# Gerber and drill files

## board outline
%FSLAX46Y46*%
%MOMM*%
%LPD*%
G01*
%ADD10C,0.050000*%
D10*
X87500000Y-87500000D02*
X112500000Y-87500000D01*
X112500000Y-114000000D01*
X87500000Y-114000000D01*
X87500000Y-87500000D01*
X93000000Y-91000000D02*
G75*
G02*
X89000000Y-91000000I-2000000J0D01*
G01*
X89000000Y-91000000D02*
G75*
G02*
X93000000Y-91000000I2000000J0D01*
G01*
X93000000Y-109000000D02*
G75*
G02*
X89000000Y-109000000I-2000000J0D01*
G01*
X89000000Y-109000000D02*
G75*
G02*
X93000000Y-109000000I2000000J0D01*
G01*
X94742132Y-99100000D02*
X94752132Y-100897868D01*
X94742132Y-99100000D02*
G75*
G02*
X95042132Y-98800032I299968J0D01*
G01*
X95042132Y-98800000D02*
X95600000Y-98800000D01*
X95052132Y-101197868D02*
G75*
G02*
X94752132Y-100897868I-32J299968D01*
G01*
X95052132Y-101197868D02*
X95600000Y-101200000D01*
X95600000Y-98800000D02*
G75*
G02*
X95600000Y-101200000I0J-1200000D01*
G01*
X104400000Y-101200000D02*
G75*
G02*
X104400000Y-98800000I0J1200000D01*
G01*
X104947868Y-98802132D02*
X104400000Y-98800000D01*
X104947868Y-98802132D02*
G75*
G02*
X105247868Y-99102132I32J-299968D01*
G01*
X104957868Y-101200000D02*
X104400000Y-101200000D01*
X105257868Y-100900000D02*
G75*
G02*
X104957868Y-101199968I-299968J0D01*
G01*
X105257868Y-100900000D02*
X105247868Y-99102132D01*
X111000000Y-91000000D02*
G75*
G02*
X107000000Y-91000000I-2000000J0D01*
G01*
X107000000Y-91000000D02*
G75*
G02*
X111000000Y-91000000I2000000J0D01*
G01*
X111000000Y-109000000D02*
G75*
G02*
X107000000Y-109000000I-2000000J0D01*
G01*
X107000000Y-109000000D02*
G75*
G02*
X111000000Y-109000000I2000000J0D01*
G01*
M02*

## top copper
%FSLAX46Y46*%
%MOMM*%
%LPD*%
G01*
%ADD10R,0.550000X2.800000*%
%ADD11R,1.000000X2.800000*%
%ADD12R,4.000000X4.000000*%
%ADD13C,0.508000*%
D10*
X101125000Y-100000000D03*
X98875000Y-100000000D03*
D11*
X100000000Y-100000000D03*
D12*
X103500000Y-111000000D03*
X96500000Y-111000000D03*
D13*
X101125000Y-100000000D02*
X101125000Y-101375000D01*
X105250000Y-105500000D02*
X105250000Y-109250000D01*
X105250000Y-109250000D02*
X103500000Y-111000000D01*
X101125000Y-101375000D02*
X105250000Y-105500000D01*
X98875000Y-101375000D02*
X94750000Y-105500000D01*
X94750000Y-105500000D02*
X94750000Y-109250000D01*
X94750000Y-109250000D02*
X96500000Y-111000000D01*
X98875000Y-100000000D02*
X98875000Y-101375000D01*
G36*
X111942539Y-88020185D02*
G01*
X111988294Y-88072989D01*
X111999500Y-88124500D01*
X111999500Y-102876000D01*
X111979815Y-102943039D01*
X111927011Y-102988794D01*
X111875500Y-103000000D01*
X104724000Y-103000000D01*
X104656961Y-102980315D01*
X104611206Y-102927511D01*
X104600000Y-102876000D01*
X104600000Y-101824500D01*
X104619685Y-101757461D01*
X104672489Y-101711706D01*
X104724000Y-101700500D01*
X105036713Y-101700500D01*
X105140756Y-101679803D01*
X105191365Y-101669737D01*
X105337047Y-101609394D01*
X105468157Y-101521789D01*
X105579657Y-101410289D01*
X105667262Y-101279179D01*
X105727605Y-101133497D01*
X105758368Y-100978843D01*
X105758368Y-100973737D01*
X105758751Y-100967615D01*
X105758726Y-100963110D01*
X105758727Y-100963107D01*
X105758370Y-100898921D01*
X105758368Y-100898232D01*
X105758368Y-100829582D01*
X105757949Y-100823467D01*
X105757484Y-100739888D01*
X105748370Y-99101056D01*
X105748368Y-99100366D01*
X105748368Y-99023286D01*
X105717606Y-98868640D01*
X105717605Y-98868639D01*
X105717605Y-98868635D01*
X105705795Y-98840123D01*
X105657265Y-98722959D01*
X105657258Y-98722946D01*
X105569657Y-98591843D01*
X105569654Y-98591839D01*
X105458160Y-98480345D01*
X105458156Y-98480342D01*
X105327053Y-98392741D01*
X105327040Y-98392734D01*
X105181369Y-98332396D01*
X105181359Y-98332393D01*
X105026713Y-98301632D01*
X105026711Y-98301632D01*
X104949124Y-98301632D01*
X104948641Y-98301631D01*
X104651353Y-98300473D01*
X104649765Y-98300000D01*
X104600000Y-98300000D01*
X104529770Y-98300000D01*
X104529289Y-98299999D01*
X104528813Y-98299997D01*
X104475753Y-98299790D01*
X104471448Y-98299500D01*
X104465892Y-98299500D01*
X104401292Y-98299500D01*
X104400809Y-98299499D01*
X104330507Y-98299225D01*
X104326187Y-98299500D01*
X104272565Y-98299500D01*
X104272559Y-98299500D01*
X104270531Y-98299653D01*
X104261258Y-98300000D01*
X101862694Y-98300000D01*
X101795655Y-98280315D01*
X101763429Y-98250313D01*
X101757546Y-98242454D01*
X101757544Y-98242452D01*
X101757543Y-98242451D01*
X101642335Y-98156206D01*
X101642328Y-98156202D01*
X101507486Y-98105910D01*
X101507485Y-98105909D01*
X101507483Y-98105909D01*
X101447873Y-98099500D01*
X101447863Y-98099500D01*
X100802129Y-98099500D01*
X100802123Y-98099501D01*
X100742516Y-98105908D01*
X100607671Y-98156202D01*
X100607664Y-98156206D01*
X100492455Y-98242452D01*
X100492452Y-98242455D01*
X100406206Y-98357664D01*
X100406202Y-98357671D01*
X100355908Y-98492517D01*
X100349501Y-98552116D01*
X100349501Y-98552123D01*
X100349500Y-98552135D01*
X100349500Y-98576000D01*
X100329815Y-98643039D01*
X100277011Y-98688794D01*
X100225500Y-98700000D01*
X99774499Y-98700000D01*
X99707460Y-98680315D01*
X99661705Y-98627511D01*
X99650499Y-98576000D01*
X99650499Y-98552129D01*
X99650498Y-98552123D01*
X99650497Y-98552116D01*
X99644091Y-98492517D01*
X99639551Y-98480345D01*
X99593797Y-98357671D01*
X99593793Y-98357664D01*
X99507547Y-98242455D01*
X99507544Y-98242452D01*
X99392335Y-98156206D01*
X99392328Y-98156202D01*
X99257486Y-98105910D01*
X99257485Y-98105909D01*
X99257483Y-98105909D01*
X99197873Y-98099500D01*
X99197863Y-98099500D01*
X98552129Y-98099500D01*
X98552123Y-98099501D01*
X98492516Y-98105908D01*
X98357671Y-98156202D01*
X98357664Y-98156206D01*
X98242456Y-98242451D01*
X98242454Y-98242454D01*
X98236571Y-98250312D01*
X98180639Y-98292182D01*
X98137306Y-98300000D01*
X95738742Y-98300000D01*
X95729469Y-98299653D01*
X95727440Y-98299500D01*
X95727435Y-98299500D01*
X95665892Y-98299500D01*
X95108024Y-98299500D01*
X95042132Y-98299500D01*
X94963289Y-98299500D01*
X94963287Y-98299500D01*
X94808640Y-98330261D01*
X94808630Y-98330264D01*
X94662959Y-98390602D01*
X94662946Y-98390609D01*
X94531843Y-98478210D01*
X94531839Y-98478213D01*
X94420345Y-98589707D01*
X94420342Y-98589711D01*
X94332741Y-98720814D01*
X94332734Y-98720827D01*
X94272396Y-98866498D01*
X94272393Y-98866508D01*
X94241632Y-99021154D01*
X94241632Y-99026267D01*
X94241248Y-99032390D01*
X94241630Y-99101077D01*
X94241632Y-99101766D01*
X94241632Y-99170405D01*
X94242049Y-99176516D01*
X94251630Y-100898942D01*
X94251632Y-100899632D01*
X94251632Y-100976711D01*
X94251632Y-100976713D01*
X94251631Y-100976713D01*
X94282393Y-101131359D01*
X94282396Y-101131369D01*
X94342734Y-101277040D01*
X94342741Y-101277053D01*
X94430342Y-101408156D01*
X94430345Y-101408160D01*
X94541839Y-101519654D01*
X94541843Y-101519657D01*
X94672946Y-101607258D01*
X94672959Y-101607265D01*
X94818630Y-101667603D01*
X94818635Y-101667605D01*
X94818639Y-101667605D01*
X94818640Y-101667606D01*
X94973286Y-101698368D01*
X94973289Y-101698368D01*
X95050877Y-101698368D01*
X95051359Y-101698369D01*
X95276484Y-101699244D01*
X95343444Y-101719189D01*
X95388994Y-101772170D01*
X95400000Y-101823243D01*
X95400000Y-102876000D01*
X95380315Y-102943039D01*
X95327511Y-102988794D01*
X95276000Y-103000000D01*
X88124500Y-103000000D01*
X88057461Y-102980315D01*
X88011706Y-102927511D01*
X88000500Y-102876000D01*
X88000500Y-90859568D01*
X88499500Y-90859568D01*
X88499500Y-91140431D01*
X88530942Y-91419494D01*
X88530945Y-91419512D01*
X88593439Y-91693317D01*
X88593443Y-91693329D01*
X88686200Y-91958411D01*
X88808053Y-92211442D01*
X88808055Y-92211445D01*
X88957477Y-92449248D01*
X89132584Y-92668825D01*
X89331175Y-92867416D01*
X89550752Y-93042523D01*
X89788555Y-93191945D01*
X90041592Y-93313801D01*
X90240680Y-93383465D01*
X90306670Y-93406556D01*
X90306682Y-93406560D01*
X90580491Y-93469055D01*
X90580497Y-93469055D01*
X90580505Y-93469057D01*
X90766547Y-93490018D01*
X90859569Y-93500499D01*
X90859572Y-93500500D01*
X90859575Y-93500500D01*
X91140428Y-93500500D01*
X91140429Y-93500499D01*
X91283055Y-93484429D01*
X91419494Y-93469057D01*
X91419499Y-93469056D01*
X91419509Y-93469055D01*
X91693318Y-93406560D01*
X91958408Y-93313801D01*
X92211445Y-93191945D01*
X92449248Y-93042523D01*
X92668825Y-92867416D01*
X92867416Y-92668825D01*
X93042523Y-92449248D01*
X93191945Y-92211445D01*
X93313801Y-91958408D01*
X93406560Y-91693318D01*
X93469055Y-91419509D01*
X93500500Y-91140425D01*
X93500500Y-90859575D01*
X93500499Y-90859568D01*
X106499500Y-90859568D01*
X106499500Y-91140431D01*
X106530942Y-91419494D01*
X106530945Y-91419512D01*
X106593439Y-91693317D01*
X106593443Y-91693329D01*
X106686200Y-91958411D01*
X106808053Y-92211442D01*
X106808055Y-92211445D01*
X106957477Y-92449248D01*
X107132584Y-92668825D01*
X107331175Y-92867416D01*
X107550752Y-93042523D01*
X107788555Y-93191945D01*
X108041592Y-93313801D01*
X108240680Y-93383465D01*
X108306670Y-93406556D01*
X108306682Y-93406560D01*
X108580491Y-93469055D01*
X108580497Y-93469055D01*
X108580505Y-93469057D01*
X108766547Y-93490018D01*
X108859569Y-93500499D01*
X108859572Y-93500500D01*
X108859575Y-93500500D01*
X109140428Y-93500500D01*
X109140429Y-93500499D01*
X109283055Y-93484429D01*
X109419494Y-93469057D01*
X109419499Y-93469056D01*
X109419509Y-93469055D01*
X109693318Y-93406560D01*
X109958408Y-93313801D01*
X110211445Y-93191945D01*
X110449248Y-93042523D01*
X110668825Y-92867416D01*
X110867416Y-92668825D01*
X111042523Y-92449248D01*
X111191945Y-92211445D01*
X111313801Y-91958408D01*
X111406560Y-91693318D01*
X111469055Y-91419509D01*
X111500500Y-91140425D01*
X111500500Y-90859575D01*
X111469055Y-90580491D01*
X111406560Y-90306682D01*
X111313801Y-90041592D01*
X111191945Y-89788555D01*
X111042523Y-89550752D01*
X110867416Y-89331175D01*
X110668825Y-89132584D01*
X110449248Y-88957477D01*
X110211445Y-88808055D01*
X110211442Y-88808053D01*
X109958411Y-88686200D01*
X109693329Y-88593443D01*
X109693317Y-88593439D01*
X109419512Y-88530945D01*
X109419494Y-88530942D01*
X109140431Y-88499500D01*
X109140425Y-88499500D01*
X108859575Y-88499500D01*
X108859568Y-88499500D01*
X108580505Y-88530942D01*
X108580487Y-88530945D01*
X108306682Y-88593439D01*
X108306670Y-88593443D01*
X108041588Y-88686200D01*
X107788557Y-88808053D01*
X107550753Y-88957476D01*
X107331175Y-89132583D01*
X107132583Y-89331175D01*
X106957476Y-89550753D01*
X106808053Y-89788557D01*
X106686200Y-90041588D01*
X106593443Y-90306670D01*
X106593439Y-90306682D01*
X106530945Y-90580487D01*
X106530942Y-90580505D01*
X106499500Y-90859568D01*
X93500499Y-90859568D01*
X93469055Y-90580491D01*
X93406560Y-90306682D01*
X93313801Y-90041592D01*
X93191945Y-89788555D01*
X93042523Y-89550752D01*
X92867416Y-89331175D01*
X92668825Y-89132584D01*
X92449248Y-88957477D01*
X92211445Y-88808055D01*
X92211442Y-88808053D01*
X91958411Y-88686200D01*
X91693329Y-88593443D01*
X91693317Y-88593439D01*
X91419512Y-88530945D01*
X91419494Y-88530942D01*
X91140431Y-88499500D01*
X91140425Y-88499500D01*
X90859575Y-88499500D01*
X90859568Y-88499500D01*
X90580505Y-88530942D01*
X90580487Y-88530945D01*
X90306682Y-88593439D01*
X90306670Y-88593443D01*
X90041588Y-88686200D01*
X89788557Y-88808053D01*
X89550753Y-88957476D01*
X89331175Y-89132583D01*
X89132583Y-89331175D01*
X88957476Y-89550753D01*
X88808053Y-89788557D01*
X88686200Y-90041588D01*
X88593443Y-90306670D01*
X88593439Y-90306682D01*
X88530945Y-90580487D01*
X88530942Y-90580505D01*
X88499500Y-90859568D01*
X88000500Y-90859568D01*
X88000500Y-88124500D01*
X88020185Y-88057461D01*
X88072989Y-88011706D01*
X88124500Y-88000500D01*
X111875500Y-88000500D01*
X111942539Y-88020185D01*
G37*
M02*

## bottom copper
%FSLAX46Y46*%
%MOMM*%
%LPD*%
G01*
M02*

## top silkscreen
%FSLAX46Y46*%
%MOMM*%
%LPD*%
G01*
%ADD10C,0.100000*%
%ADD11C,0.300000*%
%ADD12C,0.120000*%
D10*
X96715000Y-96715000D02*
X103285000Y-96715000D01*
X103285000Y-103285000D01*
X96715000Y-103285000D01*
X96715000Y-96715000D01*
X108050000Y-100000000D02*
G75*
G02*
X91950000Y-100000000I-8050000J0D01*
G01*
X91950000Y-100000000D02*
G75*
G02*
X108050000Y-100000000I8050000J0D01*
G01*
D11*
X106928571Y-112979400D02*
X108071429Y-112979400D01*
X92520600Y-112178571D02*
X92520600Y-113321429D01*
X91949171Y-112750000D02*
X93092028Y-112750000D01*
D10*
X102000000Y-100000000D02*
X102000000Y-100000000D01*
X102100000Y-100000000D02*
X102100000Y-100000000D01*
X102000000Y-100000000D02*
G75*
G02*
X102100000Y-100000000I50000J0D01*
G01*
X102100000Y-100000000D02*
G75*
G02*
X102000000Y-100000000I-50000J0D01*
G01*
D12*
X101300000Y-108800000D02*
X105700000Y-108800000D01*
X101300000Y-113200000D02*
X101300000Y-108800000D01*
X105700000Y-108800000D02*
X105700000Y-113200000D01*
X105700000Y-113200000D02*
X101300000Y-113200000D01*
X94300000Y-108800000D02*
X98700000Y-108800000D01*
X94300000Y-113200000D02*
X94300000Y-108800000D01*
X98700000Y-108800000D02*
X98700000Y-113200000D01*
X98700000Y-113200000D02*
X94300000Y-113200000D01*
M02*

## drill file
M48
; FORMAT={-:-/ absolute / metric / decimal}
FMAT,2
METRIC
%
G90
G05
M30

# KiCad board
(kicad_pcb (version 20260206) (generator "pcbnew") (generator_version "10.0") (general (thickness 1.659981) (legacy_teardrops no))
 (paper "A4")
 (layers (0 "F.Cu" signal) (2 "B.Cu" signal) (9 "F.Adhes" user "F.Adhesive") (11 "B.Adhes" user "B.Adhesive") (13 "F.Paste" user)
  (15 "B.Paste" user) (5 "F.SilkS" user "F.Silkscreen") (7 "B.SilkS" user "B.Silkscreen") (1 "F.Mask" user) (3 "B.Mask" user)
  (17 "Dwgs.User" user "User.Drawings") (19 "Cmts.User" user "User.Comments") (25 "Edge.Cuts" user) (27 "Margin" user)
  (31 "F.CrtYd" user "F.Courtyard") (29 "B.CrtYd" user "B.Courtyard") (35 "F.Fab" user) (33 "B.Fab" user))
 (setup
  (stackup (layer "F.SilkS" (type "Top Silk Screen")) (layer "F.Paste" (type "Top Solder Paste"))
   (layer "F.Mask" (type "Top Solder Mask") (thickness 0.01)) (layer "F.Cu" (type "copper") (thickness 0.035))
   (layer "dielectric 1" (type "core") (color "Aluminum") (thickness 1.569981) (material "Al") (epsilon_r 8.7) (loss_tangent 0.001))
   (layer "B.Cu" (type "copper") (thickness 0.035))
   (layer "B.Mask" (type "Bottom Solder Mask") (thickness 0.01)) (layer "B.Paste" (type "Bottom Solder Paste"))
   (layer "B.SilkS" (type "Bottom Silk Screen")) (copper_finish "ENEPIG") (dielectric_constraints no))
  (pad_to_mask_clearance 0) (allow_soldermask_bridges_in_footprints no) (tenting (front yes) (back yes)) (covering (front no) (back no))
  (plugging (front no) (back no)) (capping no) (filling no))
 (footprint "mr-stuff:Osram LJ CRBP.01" (layer "F.Cu") (at 100 100 -90)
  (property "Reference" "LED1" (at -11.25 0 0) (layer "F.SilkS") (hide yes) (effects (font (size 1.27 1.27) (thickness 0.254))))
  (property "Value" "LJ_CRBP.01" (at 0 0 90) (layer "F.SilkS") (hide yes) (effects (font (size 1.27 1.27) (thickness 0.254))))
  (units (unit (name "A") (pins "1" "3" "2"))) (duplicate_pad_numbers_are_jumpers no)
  (fp_line (start 0 -2) (end 0 -2) (stroke (width 0.1) (type solid)) (layer "F.SilkS"))
  (fp_line (start 0 -2.1) (end 0 -2.1) (stroke (width 0.1) (type solid)) (layer "F.SilkS"))
  (fp_arc (start 0 -2) (mid -0.05 -2.05) (end 0 -2.1) (stroke (width 0.1) (type solid)) (layer "F.SilkS"))
  (fp_arc (start 0 -2.1) (mid 0.05 -2.05) (end 0 -2) (stroke (width 0.1) (type solid)) (layer "F.SilkS"))
  (pad "1" smd rect (at 0 -1.125) (size 0.55 2.8) (layers "F.Cu" "F.Mask" "F.Paste") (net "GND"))
  (pad "2" smd rect (at 0 1.125) (size 0.55 2.8) (layers "F.Cu" "F.Mask" "F.Paste") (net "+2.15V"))
  (pad "3" smd rect (at 0 0) (size 1 2.8) (layers "F.Cu" "F.Mask" "F.Paste") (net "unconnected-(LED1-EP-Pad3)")))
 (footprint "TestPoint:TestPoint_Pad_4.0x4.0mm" (layer "F.Cu") (at 103.5 111)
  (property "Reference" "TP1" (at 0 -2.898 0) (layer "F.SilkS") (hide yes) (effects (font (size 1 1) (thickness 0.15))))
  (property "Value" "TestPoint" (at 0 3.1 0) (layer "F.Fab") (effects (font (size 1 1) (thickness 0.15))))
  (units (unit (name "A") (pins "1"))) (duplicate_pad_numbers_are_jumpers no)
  (fp_line (start -2.2 -2.2) (end 2.2 -2.2) (stroke (width 0.12) (type solid)) (layer "F.SilkS"))
  (fp_line (start -2.2 2.2) (end -2.2 -2.2) (stroke (width 0.12) (type solid)) (layer "F.SilkS"))
  (fp_line (start 2.2 -2.2) (end 2.2 2.2) (stroke (width 0.12) (type solid)) (layer "F.SilkS"))
  (fp_line (start 2.2 2.2) (end -2.2 2.2) (stroke (width 0.12) (type solid)) (layer "F.SilkS"))
  (pad "1" smd rect (at 0 0) (size 4 4) (layers "F.Cu" "F.Mask") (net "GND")))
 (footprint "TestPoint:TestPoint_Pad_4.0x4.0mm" (layer "F.Cu") (at 96.5 111)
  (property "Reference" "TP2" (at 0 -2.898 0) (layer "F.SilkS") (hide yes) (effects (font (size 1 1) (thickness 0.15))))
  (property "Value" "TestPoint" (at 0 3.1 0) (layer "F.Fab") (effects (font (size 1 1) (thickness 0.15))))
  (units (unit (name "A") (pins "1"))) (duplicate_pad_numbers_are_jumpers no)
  (fp_line (start -2.2 -2.2) (end 2.2 -2.2) (stroke (width 0.12) (type solid)) (layer "F.SilkS"))
  (fp_line (start -2.2 2.2) (end -2.2 -2.2) (stroke (width 0.12) (type solid)) (layer "F.SilkS"))
  (fp_line (start 2.2 -2.2) (end 2.2 2.2) (stroke (width 0.12) (type solid)) (layer "F.SilkS"))
  (fp_line (start 2.2 2.2) (end -2.2 2.2) (stroke (width 0.12) (type solid)) (layer "F.SilkS"))
  (pad "1" smd rect (at 0 0) (size 4 4) (layers "F.Cu" "F.Mask") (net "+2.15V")))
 (gr_rect (start 96.715 96.715) (end 103.285 103.285) (stroke (width 0.1) (type default)) (fill no) (layer "F.SilkS"))
 (gr_circle (center 100 100) (end 108.05 100) (stroke (width 0.1) (type default)) (fill no) (layer "F.SilkS"))
 (gr_rect (start 87.5 87.5) (end 112.5 114) (stroke (width 0.05) (type solid)) (fill no) (layer "Edge.Cuts"))
 (gr_circle (center 91 91) (end 91 93) (stroke (width 0.05) (type solid)) (fill no) (layer "Edge.Cuts"))
 (gr_circle (center 91 109) (end 91 111) (stroke (width 0.05) (type solid)) (fill no) (layer "Edge.Cuts"))
 (gr_line (start 94.742132 99.1) (end 94.752132 100.897868) (stroke (width 0.05) (type default)) (layer "Edge.Cuts"))
 (gr_arc (start 94.742132 99.1) (mid 94.83 98.887868) (end 95.042132 98.8) (stroke (width 0.05) (type default)) (layer "Edge.Cuts"))
 (gr_line (start 95.042132 98.8) (end 95.6 98.8) (stroke (width 0.05) (type default)) (layer "Edge.Cuts"))
 (gr_arc (start 95.052132 101.197868) (mid 94.84 101.11) (end 94.752132 100.897868) (stroke (width 0.05) (type default)) (layer "Edge.Cuts"))
 (gr_line (start 95.052132 101.197868) (end 95.6 101.2) (stroke (width 0.05) (type default)) (layer "Edge.Cuts"))
 (gr_arc (start 95.6 98.8) (mid 96.8 100) (end 95.6 101.2) (stroke (width 0.05) (type solid)) (layer "Edge.Cuts"))
 (gr_arc (start 104.4 101.2) (mid 103.2 100) (end 104.4 98.8) (stroke (width 0.05) (type solid)) (layer "Edge.Cuts"))
 (gr_line (start 104.947868 98.802132) (end 104.4 98.8) (stroke (width 0.05) (type default)) (layer "Edge.Cuts"))
 (gr_arc (start 104.947868 98.802132) (mid 105.16 98.89) (end 105.247868 99.102132) (stroke (width 0.05) (type default)) (layer "Edge.Cuts"))
 (gr_line (start 104.957868 101.2) (end 104.4 101.2) (stroke (width 0.05) (type default)) (layer "Edge.Cuts"))
 (gr_arc (start 105.257868 100.9) (mid 105.17 101.112132) (end 104.957868 101.2) (stroke (width 0.05) (type default)) (layer "Edge.Cuts"))
 (gr_line (start 105.257868 100.9) (end 105.247868 99.102132) (stroke (width 0.05) (type default)) (layer "Edge.Cuts"))
 (gr_circle (center 109 91) (end 109 93) (stroke (width 0.05) (type solid)) (fill no) (layer "Edge.Cuts"))
 (gr_circle (center 109 109) (end 109 111) (stroke (width 0.05) (type solid)) (fill no) (layer "Edge.Cuts"))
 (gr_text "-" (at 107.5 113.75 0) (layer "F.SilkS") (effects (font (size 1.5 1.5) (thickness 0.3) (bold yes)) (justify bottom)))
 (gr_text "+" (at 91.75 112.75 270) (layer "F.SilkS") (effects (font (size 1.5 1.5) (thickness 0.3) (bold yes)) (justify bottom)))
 (segment (start 101.125 100) (end 101.125 101.375) (width 0.508) (layer "F.Cu") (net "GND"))
 (segment (start 105.25 105.5) (end 105.25 109.25) (width 0.508) (layer "F.Cu") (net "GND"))
 (segment (start 105.25 109.25) (end 103.5 111) (width 0.508) (layer "F.Cu") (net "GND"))
 (segment (start 101.125 101.375) (end 105.25 105.5) (width 0.508) (layer "F.Cu") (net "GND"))
 (segment (start 98.875 101.375) (end 94.75 105.5) (width 0.508) (layer "F.Cu") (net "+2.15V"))
 (segment (start 94.75 105.5) (end 94.75 109.25) (width 0.508) (layer "F.Cu") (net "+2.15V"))
 (segment (start 94.75 109.25) (end 96.5 111) (width 0.508) (layer "F.Cu") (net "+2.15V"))
 (segment (start 98.875 100) (end 98.875 101.375) (width 0.508) (layer "F.Cu") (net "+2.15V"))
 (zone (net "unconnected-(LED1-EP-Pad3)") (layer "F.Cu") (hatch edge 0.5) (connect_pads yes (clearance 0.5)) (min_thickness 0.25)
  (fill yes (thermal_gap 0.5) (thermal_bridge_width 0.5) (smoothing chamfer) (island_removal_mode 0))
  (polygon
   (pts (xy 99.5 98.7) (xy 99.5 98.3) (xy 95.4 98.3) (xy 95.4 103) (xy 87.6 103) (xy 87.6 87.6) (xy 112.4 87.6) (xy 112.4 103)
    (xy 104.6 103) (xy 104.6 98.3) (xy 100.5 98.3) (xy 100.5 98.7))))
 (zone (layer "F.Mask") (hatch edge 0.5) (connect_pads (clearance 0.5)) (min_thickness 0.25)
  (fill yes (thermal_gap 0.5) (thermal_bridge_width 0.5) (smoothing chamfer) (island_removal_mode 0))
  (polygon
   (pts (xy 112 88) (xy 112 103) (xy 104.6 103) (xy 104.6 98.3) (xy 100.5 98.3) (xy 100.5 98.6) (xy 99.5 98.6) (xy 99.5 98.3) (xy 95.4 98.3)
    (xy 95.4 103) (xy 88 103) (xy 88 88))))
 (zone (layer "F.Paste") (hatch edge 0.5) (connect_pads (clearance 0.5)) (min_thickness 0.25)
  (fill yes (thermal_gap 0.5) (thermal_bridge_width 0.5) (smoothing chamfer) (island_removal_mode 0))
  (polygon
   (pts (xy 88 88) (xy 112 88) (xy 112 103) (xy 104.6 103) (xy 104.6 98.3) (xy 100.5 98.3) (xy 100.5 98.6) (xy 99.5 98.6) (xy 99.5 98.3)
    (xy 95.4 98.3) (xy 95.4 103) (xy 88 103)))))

